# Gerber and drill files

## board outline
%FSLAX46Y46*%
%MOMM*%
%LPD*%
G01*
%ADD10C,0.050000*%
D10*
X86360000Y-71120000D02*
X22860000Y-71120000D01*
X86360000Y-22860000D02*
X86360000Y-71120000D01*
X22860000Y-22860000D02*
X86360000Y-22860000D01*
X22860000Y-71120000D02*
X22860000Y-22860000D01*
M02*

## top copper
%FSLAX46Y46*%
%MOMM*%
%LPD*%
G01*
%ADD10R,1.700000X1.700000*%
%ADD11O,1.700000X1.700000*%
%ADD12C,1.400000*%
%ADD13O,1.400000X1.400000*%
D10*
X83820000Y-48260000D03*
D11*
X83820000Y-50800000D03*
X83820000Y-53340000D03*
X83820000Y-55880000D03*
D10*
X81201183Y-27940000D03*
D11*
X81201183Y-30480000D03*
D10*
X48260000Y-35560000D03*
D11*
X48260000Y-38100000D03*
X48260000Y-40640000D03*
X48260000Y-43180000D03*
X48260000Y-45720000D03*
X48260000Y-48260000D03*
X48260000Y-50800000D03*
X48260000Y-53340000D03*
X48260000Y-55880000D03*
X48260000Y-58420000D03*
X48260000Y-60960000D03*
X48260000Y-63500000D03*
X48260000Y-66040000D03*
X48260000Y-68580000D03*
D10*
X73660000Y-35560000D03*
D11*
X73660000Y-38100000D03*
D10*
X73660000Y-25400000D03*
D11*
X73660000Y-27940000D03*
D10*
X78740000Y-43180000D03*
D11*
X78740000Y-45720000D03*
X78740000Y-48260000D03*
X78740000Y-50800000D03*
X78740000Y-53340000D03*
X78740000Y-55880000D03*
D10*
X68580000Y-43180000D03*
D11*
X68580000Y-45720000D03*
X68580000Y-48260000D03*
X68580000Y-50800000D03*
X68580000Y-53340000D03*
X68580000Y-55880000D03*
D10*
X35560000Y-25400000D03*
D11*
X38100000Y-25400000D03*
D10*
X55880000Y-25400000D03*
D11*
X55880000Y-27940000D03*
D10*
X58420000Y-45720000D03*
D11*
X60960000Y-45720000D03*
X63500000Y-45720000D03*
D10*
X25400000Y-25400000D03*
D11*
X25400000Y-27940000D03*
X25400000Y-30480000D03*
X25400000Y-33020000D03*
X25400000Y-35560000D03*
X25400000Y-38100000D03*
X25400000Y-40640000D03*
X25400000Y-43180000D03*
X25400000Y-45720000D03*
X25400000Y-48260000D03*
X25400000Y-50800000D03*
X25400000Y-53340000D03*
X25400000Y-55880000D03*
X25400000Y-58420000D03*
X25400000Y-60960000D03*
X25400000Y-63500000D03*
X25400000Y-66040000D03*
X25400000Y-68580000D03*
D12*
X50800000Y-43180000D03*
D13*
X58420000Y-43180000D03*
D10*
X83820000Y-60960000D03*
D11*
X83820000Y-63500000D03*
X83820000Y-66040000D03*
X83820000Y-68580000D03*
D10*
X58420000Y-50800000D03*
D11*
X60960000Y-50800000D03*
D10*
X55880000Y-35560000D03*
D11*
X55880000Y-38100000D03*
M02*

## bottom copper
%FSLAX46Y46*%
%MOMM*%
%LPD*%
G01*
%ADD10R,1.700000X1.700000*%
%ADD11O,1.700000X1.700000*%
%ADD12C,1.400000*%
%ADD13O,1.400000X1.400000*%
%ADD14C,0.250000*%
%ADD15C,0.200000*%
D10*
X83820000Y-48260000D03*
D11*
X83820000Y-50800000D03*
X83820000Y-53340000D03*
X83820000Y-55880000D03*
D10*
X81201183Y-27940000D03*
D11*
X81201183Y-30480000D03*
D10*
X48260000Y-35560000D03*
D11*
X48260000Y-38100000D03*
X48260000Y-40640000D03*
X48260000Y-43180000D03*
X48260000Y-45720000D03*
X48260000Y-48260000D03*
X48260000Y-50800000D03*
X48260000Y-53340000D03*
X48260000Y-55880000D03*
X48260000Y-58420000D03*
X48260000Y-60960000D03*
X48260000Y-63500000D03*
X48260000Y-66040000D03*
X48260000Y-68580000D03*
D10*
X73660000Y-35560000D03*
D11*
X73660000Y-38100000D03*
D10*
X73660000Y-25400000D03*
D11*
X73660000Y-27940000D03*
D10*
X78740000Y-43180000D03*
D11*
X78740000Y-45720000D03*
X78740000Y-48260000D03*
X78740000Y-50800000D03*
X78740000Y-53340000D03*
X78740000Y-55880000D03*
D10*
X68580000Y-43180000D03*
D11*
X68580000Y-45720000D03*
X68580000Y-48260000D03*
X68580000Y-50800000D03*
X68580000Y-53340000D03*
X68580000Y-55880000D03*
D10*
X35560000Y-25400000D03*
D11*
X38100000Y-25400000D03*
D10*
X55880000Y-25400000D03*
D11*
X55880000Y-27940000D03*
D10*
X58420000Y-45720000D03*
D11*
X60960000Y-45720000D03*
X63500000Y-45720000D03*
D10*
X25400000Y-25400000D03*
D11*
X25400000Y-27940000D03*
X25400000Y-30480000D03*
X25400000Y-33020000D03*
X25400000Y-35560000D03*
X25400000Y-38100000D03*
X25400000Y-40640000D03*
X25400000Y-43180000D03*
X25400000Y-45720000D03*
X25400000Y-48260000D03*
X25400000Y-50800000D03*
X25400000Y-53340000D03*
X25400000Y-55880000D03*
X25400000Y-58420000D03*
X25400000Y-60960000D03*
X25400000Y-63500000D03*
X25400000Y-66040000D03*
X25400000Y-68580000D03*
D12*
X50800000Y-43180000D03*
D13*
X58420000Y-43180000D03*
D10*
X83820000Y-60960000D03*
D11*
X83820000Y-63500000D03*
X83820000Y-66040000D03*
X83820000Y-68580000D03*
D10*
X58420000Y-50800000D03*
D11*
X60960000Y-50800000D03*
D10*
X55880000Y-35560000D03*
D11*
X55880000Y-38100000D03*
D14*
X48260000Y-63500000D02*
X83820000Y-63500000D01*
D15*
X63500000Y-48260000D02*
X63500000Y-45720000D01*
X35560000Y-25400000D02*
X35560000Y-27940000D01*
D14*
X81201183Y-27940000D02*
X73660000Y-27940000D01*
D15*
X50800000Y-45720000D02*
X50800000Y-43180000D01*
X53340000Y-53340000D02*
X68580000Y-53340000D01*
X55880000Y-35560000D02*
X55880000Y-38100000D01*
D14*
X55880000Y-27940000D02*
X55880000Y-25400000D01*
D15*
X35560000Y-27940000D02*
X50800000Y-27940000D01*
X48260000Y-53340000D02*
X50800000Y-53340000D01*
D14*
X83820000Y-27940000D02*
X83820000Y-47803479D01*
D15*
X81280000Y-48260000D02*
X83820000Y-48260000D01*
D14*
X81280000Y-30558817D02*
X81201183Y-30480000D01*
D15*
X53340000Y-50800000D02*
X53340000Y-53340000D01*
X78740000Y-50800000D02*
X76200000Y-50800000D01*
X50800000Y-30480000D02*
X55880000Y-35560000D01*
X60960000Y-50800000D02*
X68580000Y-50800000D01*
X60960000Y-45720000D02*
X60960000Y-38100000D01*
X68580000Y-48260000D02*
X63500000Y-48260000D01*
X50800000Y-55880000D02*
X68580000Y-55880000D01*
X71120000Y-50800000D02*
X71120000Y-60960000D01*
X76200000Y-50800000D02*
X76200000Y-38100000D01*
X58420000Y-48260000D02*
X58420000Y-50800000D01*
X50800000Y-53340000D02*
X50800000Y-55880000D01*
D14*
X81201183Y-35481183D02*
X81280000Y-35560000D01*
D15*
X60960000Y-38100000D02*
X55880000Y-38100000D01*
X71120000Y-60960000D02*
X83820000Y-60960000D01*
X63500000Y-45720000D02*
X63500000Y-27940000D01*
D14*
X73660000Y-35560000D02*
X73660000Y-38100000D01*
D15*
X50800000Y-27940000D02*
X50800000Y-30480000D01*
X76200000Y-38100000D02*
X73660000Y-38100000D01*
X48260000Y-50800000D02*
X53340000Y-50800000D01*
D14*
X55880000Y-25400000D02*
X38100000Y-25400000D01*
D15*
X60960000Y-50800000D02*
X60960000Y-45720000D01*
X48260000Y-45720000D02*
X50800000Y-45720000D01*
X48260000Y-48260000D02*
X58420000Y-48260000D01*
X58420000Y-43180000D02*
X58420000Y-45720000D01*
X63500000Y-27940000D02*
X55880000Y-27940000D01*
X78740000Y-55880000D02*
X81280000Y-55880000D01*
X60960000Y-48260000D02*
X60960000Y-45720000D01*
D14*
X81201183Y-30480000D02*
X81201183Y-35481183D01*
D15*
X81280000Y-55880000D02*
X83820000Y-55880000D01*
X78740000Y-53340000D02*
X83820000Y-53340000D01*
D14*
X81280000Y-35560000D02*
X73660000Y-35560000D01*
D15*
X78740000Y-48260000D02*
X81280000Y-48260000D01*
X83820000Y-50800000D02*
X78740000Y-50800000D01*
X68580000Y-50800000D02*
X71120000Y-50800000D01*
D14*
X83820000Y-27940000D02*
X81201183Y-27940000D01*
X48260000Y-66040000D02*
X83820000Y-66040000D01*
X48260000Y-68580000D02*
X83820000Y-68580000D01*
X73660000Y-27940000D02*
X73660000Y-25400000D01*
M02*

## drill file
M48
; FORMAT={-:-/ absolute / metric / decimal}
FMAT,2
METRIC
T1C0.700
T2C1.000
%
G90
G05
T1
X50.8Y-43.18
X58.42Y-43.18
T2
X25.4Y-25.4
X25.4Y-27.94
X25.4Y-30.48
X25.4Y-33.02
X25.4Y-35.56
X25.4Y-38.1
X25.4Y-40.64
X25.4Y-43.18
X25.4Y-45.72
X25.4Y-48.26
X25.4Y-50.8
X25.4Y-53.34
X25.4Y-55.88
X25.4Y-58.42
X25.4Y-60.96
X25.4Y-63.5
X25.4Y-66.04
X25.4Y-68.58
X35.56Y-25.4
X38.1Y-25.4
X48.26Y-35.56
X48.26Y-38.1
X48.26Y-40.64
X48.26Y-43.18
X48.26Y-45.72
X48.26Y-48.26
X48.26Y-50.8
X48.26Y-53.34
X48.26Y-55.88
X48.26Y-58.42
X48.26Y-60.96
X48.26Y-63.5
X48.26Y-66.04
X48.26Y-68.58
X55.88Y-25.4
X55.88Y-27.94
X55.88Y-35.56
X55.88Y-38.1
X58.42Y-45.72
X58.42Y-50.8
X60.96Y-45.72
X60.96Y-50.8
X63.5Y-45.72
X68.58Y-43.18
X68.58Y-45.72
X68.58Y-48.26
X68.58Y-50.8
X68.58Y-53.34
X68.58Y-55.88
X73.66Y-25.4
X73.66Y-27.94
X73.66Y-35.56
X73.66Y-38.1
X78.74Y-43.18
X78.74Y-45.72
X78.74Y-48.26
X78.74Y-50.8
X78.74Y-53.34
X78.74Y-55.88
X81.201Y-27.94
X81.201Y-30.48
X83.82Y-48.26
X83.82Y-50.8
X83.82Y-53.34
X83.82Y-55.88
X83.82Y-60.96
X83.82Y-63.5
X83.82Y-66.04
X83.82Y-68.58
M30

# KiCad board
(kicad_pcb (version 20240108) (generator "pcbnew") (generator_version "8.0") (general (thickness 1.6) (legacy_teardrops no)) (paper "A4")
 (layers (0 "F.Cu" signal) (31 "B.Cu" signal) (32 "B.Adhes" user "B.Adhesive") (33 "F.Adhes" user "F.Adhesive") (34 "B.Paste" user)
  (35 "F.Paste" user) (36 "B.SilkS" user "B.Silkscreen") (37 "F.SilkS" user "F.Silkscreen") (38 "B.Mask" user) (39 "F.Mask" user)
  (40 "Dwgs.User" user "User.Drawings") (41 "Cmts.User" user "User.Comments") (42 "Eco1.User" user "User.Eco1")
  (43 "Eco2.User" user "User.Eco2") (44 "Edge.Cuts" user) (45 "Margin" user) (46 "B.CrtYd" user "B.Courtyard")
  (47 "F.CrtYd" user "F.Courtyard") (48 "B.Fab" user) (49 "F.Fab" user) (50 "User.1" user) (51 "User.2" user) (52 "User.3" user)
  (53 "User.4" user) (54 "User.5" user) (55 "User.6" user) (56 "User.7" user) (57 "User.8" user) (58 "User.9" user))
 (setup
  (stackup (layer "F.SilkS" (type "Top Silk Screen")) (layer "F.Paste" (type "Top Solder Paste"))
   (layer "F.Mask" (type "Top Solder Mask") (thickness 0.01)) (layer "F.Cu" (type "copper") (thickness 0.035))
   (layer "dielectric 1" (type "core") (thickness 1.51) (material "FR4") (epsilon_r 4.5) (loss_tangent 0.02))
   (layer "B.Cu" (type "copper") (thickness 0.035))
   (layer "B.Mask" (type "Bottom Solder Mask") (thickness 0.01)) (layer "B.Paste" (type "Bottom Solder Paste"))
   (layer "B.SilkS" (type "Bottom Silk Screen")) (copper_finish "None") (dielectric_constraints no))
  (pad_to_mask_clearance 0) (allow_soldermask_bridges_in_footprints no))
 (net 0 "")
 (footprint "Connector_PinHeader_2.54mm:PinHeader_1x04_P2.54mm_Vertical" (layer "F.Cu") (at 83.82 48.26)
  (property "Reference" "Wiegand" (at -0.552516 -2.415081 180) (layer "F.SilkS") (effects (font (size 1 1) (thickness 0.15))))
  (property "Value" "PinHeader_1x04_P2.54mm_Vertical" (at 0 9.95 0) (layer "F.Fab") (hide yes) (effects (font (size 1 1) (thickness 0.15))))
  (pad "1" thru_hole rect (at 0 0) (size 1.7 1.7) (drill 1) (layers "*.Cu" "*.Mask") (remove_unused_layers no))
  (pad "2" thru_hole oval (at 0 2.54) (size 1.7 1.7) (drill 1) (layers "*.Cu" "*.Mask") (remove_unused_layers no))
  (pad "3" thru_hole oval (at 0 5.08) (size 1.7 1.7) (drill 1) (layers "*.Cu" "*.Mask") (remove_unused_layers no))
  (pad "4" thru_hole oval (at 0 7.62) (size 1.7 1.7) (drill 1) (layers "*.Cu" "*.Mask") (remove_unused_layers no)))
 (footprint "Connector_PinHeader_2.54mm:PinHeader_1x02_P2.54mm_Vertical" (layer "F.Cu") (at 81.201183 27.94)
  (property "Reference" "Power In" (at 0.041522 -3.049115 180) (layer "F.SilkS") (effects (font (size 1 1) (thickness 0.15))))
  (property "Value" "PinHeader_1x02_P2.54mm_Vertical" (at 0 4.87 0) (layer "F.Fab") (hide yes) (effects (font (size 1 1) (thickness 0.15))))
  (pad "1" thru_hole rect (at 0 0) (size 1.7 1.7) (drill 1) (layers "*.Cu" "*.Mask") (remove_unused_layers no))
  (pad "2" thru_hole oval (at 0 2.54) (size 1.7 1.7) (drill 1) (layers "*.Cu" "*.Mask") (remove_unused_layers no)))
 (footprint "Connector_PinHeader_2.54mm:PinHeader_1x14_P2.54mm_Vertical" (layer "F.Cu") (at 48.26 35.56)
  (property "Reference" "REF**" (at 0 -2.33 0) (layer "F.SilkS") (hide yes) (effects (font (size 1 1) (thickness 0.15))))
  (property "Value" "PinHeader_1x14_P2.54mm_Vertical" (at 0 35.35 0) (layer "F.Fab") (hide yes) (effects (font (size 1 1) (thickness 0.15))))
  (pad "1" thru_hole rect (at 0 0) (size 1.7 1.7) (drill 1) (layers "*.Cu" "*.Mask") (remove_unused_layers no))
  (pad "2" thru_hole oval (at 0 2.54) (size 1.7 1.7) (drill 1) (layers "*.Cu" "*.Mask") (remove_unused_layers no))
  (pad "3" thru_hole oval (at 0 5.08) (size 1.7 1.7) (drill 1) (layers "*.Cu" "*.Mask") (remove_unused_layers no))
  (pad "4" thru_hole oval (at 0 7.62) (size 1.7 1.7) (drill 1) (layers "*.Cu" "*.Mask") (remove_unused_layers no))
  (pad "5" thru_hole oval (at 0 10.16) (size 1.7 1.7) (drill 1) (layers "*.Cu" "*.Mask") (remove_unused_layers no))
  (pad "6" thru_hole oval (at 0 12.7) (size 1.7 1.7) (drill 1) (layers "*.Cu" "*.Mask") (remove_unused_layers no))
  (pad "7" thru_hole oval (at 0 15.24) (size 1.7 1.7) (drill 1) (layers "*.Cu" "*.Mask") (remove_unused_layers no))
  (pad "8" thru_hole oval (at 0 17.78) (size 1.7 1.7) (drill 1) (layers "*.Cu" "*.Mask") (remove_unused_layers no))
  (pad "9" thru_hole oval (at 0 20.32) (size 1.7 1.7) (drill 1) (layers "*.Cu" "*.Mask") (remove_unused_layers no))
  (pad "10" thru_hole oval (at 0 22.86) (size 1.7 1.7) (drill 1) (layers "*.Cu" "*.Mask") (remove_unused_layers no))
  (pad "11" thru_hole oval (at 0 25.4) (size 1.7 1.7) (drill 1) (layers "*.Cu" "*.Mask") (remove_unused_layers no))
  (pad "12" thru_hole oval (at 0 27.94) (size 1.7 1.7) (drill 1) (layers "*.Cu" "*.Mask") (remove_unused_layers no))
  (pad "13" thru_hole oval (at 0 30.48) (size 1.7 1.7) (drill 1) (layers "*.Cu" "*.Mask") (remove_unused_layers no))
  (pad "14" thru_hole oval (at 0 33.02) (size 1.7 1.7) (drill 1) (layers "*.Cu" "*.Mask") (remove_unused_layers no)))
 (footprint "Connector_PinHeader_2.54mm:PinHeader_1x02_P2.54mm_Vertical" (layer "F.Cu") (at 73.66 35.56)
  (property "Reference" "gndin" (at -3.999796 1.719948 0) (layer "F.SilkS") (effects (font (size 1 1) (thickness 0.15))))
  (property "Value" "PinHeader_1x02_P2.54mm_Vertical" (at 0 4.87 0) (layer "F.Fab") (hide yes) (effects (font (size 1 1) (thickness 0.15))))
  (pad "1" thru_hole rect (at 0 0) (size 1.7 1.7) (drill 1) (layers "*.Cu" "*.Mask") (remove_unused_layers no))
  (pad "2" thru_hole oval (at 0 2.54) (size 1.7 1.7) (drill 1) (layers "*.Cu" "*.Mask") (remove_unused_layers no)))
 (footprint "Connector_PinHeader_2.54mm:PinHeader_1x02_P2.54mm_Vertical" (layer "F.Cu") (at 73.66 25.4)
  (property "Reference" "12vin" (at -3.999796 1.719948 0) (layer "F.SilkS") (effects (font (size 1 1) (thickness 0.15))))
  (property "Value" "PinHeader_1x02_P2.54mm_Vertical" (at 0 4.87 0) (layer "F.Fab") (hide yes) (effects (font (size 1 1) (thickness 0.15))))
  (pad "1" thru_hole rect (at 0 0) (size 1.7 1.7) (drill 1) (layers "*.Cu" "*.Mask") (remove_unused_layers no))
  (pad "2" thru_hole oval (at 0 2.54) (size 1.7 1.7) (drill 1) (layers "*.Cu" "*.Mask") (remove_unused_layers no)))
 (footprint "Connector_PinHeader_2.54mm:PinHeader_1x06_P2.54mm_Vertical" (layer "F.Cu") (at 78.74 43.18)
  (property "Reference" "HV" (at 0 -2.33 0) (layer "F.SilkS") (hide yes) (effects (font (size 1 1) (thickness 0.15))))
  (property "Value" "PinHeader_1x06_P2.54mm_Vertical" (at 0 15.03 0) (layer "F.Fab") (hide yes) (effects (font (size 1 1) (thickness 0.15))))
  (pad "1" thru_hole rect (at 0 0) (size 1.7 1.7) (drill 1) (layers "*.Cu" "*.Mask") (remove_unused_layers no))
  (pad "2" thru_hole oval (at 0 2.54) (size 1.7 1.7) (drill 1) (layers "*.Cu" "*.Mask") (remove_unused_layers no))
  (pad "3" thru_hole oval (at 0 5.08) (size 1.7 1.7) (drill 1) (layers "*.Cu" "*.Mask") (remove_unused_layers no))
  (pad "4" thru_hole oval (at 0 7.62) (size 1.7 1.7) (drill 1) (layers "*.Cu" "*.Mask") (remove_unused_layers no))
  (pad "5" thru_hole oval (at 0 10.16) (size 1.7 1.7) (drill 1) (layers "*.Cu" "*.Mask") (remove_unused_layers no))
  (pad "6" thru_hole oval (at 0 12.7) (size 1.7 1.7) (drill 1) (layers "*.Cu" "*.Mask") (remove_unused_layers no)))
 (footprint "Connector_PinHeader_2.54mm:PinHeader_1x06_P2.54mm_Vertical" (layer "F.Cu") (at 68.58 43.18)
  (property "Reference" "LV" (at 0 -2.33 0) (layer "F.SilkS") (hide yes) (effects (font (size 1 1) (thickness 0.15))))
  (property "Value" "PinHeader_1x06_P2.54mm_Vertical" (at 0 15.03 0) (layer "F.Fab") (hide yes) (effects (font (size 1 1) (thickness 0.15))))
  (pad "1" thru_hole rect (at 0 0) (size 1.7 1.7) (drill 1) (layers "*.Cu" "*.Mask") (remove_unused_layers no))
  (pad "2" thru_hole oval (at 0 2.54) (size 1.7 1.7) (drill 1) (layers "*.Cu" "*.Mask") (remove_unused_layers no))
  (pad "3" thru_hole oval (at 0 5.08) (size 1.7 1.7) (drill 1) (layers "*.Cu" "*.Mask") (remove_unused_layers no))
  (pad "4" thru_hole oval (at 0 7.62) (size 1.7 1.7) (drill 1) (layers "*.Cu" "*.Mask") (remove_unused_layers no))
  (pad "5" thru_hole oval (at 0 10.16) (size 1.7 1.7) (drill 1) (layers "*.Cu" "*.Mask") (remove_unused_layers no))
  (pad "6" thru_hole oval (at 0 12.7) (size 1.7 1.7) (drill 1) (layers "*.Cu" "*.Mask") (remove_unused_layers no)))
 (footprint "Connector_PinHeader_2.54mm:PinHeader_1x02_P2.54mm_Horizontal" (layer "F.Cu") (at 35.56 25.4 90)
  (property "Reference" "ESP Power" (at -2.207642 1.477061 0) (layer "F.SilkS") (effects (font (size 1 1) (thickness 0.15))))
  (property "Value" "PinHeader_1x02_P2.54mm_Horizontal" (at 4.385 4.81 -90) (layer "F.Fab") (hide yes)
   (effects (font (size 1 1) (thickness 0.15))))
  (pad "1" thru_hole rect (at 0 0 90) (size 1.7 1.7) (drill 1) (layers "*.Cu" "*.Mask") (remove_unused_layers no))
  (pad "2" thru_hole oval (at 0 2.54 90) (size 1.7 1.7) (drill 1) (layers "*.Cu" "*.Mask") (remove_unused_layers no)))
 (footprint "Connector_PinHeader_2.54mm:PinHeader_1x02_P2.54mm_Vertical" (layer "F.Cu") (at 55.88 25.4)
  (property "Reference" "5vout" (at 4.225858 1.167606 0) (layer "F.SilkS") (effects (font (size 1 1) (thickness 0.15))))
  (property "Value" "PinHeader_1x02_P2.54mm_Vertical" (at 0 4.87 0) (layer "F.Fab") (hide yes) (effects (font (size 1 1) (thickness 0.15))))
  (pad "1" thru_hole rect (at 0 0) (size 1.7 1.7) (drill 1) (layers "*.Cu" "*.Mask") (remove_unused_layers no))
  (pad "2" thru_hole oval (at 0 2.54) (size 1.7 1.7) (drill 1) (layers "*.Cu" "*.Mask") (remove_unused_layers no)))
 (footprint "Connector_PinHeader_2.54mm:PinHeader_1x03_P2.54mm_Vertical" (layer "F.Cu") (at 58.42 45.72 90)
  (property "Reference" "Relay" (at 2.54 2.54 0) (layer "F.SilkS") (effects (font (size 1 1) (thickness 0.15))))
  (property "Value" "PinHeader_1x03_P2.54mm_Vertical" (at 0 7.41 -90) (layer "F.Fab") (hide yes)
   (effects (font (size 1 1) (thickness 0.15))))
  (pad "1" thru_hole rect (at 0 0 90) (size 1.7 1.7) (drill 1) (layers "*.Cu" "*.Mask") (remove_unused_layers no))
  (pad "2" thru_hole oval (at 0 2.54 90) (size 1.7 1.7) (drill 1) (layers "*.Cu" "*.Mask") (remove_unused_layers no))
  (pad "3" thru_hole oval (at 0 5.08 90) (size 1.7 1.7) (drill 1) (layers "*.Cu" "*.Mask") (remove_unused_layers no)))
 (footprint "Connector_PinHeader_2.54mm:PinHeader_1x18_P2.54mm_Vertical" (layer "F.Cu") (at 25.4 25.4)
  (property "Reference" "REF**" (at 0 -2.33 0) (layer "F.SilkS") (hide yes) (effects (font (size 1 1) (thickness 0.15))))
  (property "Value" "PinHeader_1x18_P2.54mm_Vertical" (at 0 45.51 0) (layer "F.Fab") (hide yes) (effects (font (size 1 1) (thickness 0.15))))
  (pad "1" thru_hole rect (at 0 0) (size 1.7 1.7) (drill 1) (layers "*.Cu" "*.Mask") (remove_unused_layers no))
  (pad "2" thru_hole oval (at 0 2.54) (size 1.7 1.7) (drill 1) (layers "*.Cu" "*.Mask") (remove_unused_layers no))
  (pad "3" thru_hole oval (at 0 5.08) (size 1.7 1.7) (drill 1) (layers "*.Cu" "*.Mask") (remove_unused_layers no))
  (pad "4" thru_hole oval (at 0 7.62) (size 1.7 1.7) (drill 1) (layers "*.Cu" "*.Mask") (remove_unused_layers no))
  (pad "5" thru_hole oval (at 0 10.16) (size 1.7 1.7) (drill 1) (layers "*.Cu" "*.Mask") (remove_unused_layers no))
  (pad "6" thru_hole oval (at 0 12.7) (size 1.7 1.7) (drill 1) (layers "*.Cu" "*.Mask") (remove_unused_layers no))
  (pad "7" thru_hole oval (at 0 15.24) (size 1.7 1.7) (drill 1) (layers "*.Cu" "*.Mask") (remove_unused_layers no))
  (pad "8" thru_hole oval (at 0 17.78) (size 1.7 1.7) (drill 1) (layers "*.Cu" "*.Mask") (remove_unused_layers no))
  (pad "9" thru_hole oval (at 0 20.32) (size 1.7 1.7) (drill 1) (layers "*.Cu" "*.Mask") (remove_unused_layers no))
  (pad "10" thru_hole oval (at 0 22.86) (size 1.7 1.7) (drill 1) (layers "*.Cu" "*.Mask") (remove_unused_layers no))
  (pad "11" thru_hole oval (at 0 25.4) (size 1.7 1.7) (drill 1) (layers "*.Cu" "*.Mask") (remove_unused_layers no))
  (pad "12" thru_hole oval (at 0 27.94) (size 1.7 1.7) (drill 1) (layers "*.Cu" "*.Mask") (remove_unused_layers no))
  (pad "13" thru_hole oval (at 0 30.48) (size 1.7 1.7) (drill 1) (layers "*.Cu" "*.Mask") (remove_unused_layers no))
  (pad "14" thru_hole oval (at 0 33.02) (size 1.7 1.7) (drill 1) (layers "*.Cu" "*.Mask") (remove_unused_layers no))
  (pad "15" thru_hole oval (at 0 35.56) (size 1.7 1.7) (drill 1) (layers "*.Cu" "*.Mask") (remove_unused_layers no))
  (pad "16" thru_hole oval (at 0 38.1) (size 1.7 1.7) (drill 1) (layers "*.Cu" "*.Mask") (remove_unused_layers no))
  (pad "17" thru_hole oval (at 0 40.64) (size 1.7 1.7) (drill 1) (layers "*.Cu" "*.Mask") (remove_unused_layers no))
  (pad "18" thru_hole oval (at 0 43.18) (size 1.7 1.7) (drill 1) (layers "*.Cu" "*.Mask") (remove_unused_layers no)))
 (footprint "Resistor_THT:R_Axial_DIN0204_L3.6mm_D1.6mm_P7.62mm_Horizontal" (layer "F.Cu") (at 50.8 43.18)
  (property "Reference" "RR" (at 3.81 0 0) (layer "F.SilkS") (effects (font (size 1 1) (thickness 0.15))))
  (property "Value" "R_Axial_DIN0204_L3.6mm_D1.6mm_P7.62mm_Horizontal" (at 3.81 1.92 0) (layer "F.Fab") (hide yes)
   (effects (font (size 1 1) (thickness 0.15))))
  (pad "1" thru_hole circle (at 0 0) (size 1.4 1.4) (drill 0.7) (layers "*.Cu" "*.Mask") (remove_unused_layers no))
  (pad "2" thru_hole oval (at 7.62 0) (size 1.4 1.4) (drill 0.7) (layers "*.Cu" "*.Mask") (remove_unused_layers no)))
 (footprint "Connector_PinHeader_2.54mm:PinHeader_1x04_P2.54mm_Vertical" (layer "F.Cu") (at 83.82 60.96)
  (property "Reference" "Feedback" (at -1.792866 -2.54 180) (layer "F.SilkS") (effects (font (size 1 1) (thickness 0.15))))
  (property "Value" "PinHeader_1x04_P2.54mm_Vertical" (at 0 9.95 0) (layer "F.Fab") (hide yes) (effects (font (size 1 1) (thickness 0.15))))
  (pad "1" thru_hole rect (at 0 0) (size 1.7 1.7) (drill 1) (layers "*.Cu" "*.Mask") (remove_unused_layers no))
  (pad "2" thru_hole oval (at 0 2.54) (size 1.7 1.7) (drill 1) (layers "*.Cu" "*.Mask") (remove_unused_layers no))
  (pad "3" thru_hole oval (at 0 5.08) (size 1.7 1.7) (drill 1) (layers "*.Cu" "*.Mask") (remove_unused_layers no))
  (pad "4" thru_hole oval (at 0 7.62) (size 1.7 1.7) (drill 1) (layers "*.Cu" "*.Mask") (remove_unused_layers no)))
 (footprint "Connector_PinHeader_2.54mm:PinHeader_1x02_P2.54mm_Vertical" (layer "F.Cu") (at 58.42 50.8 90)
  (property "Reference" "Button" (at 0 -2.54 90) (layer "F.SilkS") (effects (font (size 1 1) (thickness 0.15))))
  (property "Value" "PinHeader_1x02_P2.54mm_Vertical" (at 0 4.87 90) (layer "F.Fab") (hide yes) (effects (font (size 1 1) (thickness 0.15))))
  (pad "1" thru_hole rect (at 0 0 90) (size 1.7 1.7) (drill 1) (layers "*.Cu" "*.Mask") (remove_unused_layers no))
  (pad "2" thru_hole oval (at 0 2.54 90) (size 1.7 1.7) (drill 1) (layers "*.Cu" "*.Mask") (remove_unused_layers no)))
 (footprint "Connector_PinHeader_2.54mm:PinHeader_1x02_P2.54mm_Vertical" (layer "F.Cu") (at 55.88 35.56)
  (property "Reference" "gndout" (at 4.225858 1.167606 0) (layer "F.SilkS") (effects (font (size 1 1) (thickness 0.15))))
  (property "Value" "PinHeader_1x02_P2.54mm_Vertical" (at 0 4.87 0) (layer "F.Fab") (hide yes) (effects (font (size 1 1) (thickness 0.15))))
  (pad "1" thru_hole rect (at 0 0) (size 1.7 1.7) (drill 1) (layers "*.Cu" "*.Mask") (remove_unused_layers no))
  (pad "2" thru_hole oval (at 0 2.54) (size 1.7 1.7) (drill 1) (layers "*.Cu" "*.Mask") (remove_unused_layers no)))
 (gr_line (start 86.36 71.12) (end 22.86 71.12) (stroke (width 0.05) (type default)) (layer "Edge.Cuts"))
 (gr_line (start 86.36 22.86) (end 86.36 71.12) (stroke (width 0.05) (type default)) (layer "Edge.Cuts"))
 (gr_line (start 22.86 22.86) (end 86.36 22.86) (stroke (width 0.05) (type default)) (layer "Edge.Cuts"))
 (gr_line (start 22.86 71.12) (end 22.86 22.86) (stroke (width 0.05) (type default)) (layer "Edge.Cuts"))
 (segment (start 48.26 63.5) (end 83.82 63.5) (width 0.25) (layer "B.Cu") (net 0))
 (segment (start 63.5 48.26) (end 63.5 45.72) (width 0.2) (layer "B.Cu") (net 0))
 (segment (start 35.56 25.4) (end 35.56 27.94) (width 0.2) (layer "B.Cu") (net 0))
 (segment (start 81.201183 27.94) (end 73.66 27.94) (width 0.25) (layer "B.Cu") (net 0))
 (segment (start 50.8 45.72) (end 50.8 43.18) (width 0.2) (layer "B.Cu") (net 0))
 (segment (start 53.34 53.34) (end 68.58 53.34) (width 0.2) (layer "B.Cu") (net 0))
 (segment (start 55.88 35.56) (end 55.88 38.1) (width 0.2) (layer "B.Cu") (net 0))
 (segment (start 55.88 27.94) (end 55.88 25.4) (width 0.25) (layer "B.Cu") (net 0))
 (segment (start 35.56 27.94) (end 50.8 27.94) (width 0.2) (layer "B.Cu") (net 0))
 (segment (start 48.26 53.34) (end 50.8 53.34) (width 0.2) (layer "B.Cu") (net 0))
 (segment (start 83.82 27.94) (end 83.82 47.803479) (width 0.25) (layer "B.Cu") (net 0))
 (segment (start 81.28 48.26) (end 83.82 48.26) (width 0.2) (layer "B.Cu") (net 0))
 (segment (start 81.28 30.558817) (end 81.201183 30.48) (width 0.25) (layer "B.Cu") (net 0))
 (segment (start 53.34 50.8) (end 53.34 53.34) (width 0.2) (layer "B.Cu") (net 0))
 (segment (start 78.74 50.8) (end 76.2 50.8) (width 0.2) (layer "B.Cu") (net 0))
 (segment (start 50.8 30.48) (end 55.88 35.56) (width 0.2) (layer "B.Cu") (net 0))
 (segment (start 60.96 50.8) (end 68.58 50.8) (width 0.2) (layer "B.Cu") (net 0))
 (segment (start 60.96 45.72) (end 60.96 38.1) (width 0.2) (layer "B.Cu") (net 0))
 (segment (start 68.58 48.26) (end 63.5 48.26) (width 0.2) (layer "B.Cu") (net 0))
 (segment (start 50.8 55.88) (end 68.58 55.88) (width 0.2) (layer "B.Cu") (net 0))
 (segment (start 71.12 50.8) (end 71.12 60.96) (width 0.2) (layer "B.Cu") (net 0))
 (segment (start 76.2 50.8) (end 76.2 38.1) (width 0.2) (layer "B.Cu") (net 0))
 (segment (start 58.42 48.26) (end 58.42 50.8) (width 0.2) (layer "B.Cu") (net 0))
 (segment (start 50.8 53.34) (end 50.8 55.88) (width 0.2) (layer "B.Cu") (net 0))
 (segment (start 81.201183 35.481183) (end 81.28 35.56) (width 0.25) (layer "B.Cu") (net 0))
 (segment (start 60.96 38.1) (end 55.88 38.1) (width 0.2) (layer "B.Cu") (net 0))
 (segment (start 71.12 60.96) (end 83.82 60.96) (width 0.2) (layer "B.Cu") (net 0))
 (segment (start 63.5 45.72) (end 63.5 27.94) (width 0.2) (layer "B.Cu") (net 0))
 (segment (start 73.66 35.56) (end 73.66 38.1) (width 0.25) (layer "B.Cu") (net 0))
 (segment (start 50.8 27.94) (end 50.8 30.48) (width 0.2) (layer "B.Cu") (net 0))
 (segment (start 76.2 38.1) (end 73.66 38.1) (width 0.2) (layer "B.Cu") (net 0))
 (segment (start 48.26 50.8) (end 53.34 50.8) (width 0.2) (layer "B.Cu") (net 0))
 (segment (start 55.88 25.4) (end 38.1 25.4) (width 0.25) (layer "B.Cu") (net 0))
 (segment (start 60.96 50.8) (end 60.96 45.72) (width 0.2) (layer "B.Cu") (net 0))
 (segment (start 48.26 45.72) (end 50.8 45.72) (width 0.2) (layer "B.Cu") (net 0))
 (segment (start 48.26 48.26) (end 58.42 48.26) (width 0.2) (layer "B.Cu") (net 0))
 (segment (start 58.42 43.18) (end 58.42 45.72) (width 0.2) (layer "B.Cu") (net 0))
 (segment (start 63.5 27.94) (end 55.88 27.94) (width 0.2) (layer "B.Cu") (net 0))
 (segment (start 78.74 55.88) (end 81.28 55.88) (width 0.2) (layer "B.Cu") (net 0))
 (segment (start 60.96 48.26) (end 60.96 45.72) (width 0.2) (layer "B.Cu") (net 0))
 (segment (start 81.201183 30.48) (end 81.201183 35.481183) (width 0.25) (layer "B.Cu") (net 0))
 (segment (start 81.28 55.88) (end 83.82 55.88) (width 0.2) (layer "B.Cu") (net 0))
 (segment (start 78.74 53.34) (end 83.82 53.34) (width 0.2) (layer "B.Cu") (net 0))
 (segment (start 81.28 35.56) (end 73.66 35.56) (width 0.25) (layer "B.Cu") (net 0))
 (segment (start 78.74 48.26) (end 81.28 48.26) (width 0.2) (layer "B.Cu") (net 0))
 (segment (start 83.82 50.8) (end 78.74 50.8) (width 0.2) (layer "B.Cu") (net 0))
 (segment (start 68.58 50.8) (end 71.12 50.8) (width 0.2) (layer "B.Cu") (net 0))
 (segment (start 83.82 27.94) (end 81.201183 27.94) (width 0.25) (layer "B.Cu") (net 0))
 (segment (start 48.26 66.04) (end 83.82 66.04) (width 0.25) (layer "B.Cu") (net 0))
 (segment (start 48.26 68.58) (end 83.82 68.58) (width 0.25) (layer "B.Cu") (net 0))
 (segment (start 73.66 27.94) (end 73.66 25.4) (width 0.25) (layer "B.Cu") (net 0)))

